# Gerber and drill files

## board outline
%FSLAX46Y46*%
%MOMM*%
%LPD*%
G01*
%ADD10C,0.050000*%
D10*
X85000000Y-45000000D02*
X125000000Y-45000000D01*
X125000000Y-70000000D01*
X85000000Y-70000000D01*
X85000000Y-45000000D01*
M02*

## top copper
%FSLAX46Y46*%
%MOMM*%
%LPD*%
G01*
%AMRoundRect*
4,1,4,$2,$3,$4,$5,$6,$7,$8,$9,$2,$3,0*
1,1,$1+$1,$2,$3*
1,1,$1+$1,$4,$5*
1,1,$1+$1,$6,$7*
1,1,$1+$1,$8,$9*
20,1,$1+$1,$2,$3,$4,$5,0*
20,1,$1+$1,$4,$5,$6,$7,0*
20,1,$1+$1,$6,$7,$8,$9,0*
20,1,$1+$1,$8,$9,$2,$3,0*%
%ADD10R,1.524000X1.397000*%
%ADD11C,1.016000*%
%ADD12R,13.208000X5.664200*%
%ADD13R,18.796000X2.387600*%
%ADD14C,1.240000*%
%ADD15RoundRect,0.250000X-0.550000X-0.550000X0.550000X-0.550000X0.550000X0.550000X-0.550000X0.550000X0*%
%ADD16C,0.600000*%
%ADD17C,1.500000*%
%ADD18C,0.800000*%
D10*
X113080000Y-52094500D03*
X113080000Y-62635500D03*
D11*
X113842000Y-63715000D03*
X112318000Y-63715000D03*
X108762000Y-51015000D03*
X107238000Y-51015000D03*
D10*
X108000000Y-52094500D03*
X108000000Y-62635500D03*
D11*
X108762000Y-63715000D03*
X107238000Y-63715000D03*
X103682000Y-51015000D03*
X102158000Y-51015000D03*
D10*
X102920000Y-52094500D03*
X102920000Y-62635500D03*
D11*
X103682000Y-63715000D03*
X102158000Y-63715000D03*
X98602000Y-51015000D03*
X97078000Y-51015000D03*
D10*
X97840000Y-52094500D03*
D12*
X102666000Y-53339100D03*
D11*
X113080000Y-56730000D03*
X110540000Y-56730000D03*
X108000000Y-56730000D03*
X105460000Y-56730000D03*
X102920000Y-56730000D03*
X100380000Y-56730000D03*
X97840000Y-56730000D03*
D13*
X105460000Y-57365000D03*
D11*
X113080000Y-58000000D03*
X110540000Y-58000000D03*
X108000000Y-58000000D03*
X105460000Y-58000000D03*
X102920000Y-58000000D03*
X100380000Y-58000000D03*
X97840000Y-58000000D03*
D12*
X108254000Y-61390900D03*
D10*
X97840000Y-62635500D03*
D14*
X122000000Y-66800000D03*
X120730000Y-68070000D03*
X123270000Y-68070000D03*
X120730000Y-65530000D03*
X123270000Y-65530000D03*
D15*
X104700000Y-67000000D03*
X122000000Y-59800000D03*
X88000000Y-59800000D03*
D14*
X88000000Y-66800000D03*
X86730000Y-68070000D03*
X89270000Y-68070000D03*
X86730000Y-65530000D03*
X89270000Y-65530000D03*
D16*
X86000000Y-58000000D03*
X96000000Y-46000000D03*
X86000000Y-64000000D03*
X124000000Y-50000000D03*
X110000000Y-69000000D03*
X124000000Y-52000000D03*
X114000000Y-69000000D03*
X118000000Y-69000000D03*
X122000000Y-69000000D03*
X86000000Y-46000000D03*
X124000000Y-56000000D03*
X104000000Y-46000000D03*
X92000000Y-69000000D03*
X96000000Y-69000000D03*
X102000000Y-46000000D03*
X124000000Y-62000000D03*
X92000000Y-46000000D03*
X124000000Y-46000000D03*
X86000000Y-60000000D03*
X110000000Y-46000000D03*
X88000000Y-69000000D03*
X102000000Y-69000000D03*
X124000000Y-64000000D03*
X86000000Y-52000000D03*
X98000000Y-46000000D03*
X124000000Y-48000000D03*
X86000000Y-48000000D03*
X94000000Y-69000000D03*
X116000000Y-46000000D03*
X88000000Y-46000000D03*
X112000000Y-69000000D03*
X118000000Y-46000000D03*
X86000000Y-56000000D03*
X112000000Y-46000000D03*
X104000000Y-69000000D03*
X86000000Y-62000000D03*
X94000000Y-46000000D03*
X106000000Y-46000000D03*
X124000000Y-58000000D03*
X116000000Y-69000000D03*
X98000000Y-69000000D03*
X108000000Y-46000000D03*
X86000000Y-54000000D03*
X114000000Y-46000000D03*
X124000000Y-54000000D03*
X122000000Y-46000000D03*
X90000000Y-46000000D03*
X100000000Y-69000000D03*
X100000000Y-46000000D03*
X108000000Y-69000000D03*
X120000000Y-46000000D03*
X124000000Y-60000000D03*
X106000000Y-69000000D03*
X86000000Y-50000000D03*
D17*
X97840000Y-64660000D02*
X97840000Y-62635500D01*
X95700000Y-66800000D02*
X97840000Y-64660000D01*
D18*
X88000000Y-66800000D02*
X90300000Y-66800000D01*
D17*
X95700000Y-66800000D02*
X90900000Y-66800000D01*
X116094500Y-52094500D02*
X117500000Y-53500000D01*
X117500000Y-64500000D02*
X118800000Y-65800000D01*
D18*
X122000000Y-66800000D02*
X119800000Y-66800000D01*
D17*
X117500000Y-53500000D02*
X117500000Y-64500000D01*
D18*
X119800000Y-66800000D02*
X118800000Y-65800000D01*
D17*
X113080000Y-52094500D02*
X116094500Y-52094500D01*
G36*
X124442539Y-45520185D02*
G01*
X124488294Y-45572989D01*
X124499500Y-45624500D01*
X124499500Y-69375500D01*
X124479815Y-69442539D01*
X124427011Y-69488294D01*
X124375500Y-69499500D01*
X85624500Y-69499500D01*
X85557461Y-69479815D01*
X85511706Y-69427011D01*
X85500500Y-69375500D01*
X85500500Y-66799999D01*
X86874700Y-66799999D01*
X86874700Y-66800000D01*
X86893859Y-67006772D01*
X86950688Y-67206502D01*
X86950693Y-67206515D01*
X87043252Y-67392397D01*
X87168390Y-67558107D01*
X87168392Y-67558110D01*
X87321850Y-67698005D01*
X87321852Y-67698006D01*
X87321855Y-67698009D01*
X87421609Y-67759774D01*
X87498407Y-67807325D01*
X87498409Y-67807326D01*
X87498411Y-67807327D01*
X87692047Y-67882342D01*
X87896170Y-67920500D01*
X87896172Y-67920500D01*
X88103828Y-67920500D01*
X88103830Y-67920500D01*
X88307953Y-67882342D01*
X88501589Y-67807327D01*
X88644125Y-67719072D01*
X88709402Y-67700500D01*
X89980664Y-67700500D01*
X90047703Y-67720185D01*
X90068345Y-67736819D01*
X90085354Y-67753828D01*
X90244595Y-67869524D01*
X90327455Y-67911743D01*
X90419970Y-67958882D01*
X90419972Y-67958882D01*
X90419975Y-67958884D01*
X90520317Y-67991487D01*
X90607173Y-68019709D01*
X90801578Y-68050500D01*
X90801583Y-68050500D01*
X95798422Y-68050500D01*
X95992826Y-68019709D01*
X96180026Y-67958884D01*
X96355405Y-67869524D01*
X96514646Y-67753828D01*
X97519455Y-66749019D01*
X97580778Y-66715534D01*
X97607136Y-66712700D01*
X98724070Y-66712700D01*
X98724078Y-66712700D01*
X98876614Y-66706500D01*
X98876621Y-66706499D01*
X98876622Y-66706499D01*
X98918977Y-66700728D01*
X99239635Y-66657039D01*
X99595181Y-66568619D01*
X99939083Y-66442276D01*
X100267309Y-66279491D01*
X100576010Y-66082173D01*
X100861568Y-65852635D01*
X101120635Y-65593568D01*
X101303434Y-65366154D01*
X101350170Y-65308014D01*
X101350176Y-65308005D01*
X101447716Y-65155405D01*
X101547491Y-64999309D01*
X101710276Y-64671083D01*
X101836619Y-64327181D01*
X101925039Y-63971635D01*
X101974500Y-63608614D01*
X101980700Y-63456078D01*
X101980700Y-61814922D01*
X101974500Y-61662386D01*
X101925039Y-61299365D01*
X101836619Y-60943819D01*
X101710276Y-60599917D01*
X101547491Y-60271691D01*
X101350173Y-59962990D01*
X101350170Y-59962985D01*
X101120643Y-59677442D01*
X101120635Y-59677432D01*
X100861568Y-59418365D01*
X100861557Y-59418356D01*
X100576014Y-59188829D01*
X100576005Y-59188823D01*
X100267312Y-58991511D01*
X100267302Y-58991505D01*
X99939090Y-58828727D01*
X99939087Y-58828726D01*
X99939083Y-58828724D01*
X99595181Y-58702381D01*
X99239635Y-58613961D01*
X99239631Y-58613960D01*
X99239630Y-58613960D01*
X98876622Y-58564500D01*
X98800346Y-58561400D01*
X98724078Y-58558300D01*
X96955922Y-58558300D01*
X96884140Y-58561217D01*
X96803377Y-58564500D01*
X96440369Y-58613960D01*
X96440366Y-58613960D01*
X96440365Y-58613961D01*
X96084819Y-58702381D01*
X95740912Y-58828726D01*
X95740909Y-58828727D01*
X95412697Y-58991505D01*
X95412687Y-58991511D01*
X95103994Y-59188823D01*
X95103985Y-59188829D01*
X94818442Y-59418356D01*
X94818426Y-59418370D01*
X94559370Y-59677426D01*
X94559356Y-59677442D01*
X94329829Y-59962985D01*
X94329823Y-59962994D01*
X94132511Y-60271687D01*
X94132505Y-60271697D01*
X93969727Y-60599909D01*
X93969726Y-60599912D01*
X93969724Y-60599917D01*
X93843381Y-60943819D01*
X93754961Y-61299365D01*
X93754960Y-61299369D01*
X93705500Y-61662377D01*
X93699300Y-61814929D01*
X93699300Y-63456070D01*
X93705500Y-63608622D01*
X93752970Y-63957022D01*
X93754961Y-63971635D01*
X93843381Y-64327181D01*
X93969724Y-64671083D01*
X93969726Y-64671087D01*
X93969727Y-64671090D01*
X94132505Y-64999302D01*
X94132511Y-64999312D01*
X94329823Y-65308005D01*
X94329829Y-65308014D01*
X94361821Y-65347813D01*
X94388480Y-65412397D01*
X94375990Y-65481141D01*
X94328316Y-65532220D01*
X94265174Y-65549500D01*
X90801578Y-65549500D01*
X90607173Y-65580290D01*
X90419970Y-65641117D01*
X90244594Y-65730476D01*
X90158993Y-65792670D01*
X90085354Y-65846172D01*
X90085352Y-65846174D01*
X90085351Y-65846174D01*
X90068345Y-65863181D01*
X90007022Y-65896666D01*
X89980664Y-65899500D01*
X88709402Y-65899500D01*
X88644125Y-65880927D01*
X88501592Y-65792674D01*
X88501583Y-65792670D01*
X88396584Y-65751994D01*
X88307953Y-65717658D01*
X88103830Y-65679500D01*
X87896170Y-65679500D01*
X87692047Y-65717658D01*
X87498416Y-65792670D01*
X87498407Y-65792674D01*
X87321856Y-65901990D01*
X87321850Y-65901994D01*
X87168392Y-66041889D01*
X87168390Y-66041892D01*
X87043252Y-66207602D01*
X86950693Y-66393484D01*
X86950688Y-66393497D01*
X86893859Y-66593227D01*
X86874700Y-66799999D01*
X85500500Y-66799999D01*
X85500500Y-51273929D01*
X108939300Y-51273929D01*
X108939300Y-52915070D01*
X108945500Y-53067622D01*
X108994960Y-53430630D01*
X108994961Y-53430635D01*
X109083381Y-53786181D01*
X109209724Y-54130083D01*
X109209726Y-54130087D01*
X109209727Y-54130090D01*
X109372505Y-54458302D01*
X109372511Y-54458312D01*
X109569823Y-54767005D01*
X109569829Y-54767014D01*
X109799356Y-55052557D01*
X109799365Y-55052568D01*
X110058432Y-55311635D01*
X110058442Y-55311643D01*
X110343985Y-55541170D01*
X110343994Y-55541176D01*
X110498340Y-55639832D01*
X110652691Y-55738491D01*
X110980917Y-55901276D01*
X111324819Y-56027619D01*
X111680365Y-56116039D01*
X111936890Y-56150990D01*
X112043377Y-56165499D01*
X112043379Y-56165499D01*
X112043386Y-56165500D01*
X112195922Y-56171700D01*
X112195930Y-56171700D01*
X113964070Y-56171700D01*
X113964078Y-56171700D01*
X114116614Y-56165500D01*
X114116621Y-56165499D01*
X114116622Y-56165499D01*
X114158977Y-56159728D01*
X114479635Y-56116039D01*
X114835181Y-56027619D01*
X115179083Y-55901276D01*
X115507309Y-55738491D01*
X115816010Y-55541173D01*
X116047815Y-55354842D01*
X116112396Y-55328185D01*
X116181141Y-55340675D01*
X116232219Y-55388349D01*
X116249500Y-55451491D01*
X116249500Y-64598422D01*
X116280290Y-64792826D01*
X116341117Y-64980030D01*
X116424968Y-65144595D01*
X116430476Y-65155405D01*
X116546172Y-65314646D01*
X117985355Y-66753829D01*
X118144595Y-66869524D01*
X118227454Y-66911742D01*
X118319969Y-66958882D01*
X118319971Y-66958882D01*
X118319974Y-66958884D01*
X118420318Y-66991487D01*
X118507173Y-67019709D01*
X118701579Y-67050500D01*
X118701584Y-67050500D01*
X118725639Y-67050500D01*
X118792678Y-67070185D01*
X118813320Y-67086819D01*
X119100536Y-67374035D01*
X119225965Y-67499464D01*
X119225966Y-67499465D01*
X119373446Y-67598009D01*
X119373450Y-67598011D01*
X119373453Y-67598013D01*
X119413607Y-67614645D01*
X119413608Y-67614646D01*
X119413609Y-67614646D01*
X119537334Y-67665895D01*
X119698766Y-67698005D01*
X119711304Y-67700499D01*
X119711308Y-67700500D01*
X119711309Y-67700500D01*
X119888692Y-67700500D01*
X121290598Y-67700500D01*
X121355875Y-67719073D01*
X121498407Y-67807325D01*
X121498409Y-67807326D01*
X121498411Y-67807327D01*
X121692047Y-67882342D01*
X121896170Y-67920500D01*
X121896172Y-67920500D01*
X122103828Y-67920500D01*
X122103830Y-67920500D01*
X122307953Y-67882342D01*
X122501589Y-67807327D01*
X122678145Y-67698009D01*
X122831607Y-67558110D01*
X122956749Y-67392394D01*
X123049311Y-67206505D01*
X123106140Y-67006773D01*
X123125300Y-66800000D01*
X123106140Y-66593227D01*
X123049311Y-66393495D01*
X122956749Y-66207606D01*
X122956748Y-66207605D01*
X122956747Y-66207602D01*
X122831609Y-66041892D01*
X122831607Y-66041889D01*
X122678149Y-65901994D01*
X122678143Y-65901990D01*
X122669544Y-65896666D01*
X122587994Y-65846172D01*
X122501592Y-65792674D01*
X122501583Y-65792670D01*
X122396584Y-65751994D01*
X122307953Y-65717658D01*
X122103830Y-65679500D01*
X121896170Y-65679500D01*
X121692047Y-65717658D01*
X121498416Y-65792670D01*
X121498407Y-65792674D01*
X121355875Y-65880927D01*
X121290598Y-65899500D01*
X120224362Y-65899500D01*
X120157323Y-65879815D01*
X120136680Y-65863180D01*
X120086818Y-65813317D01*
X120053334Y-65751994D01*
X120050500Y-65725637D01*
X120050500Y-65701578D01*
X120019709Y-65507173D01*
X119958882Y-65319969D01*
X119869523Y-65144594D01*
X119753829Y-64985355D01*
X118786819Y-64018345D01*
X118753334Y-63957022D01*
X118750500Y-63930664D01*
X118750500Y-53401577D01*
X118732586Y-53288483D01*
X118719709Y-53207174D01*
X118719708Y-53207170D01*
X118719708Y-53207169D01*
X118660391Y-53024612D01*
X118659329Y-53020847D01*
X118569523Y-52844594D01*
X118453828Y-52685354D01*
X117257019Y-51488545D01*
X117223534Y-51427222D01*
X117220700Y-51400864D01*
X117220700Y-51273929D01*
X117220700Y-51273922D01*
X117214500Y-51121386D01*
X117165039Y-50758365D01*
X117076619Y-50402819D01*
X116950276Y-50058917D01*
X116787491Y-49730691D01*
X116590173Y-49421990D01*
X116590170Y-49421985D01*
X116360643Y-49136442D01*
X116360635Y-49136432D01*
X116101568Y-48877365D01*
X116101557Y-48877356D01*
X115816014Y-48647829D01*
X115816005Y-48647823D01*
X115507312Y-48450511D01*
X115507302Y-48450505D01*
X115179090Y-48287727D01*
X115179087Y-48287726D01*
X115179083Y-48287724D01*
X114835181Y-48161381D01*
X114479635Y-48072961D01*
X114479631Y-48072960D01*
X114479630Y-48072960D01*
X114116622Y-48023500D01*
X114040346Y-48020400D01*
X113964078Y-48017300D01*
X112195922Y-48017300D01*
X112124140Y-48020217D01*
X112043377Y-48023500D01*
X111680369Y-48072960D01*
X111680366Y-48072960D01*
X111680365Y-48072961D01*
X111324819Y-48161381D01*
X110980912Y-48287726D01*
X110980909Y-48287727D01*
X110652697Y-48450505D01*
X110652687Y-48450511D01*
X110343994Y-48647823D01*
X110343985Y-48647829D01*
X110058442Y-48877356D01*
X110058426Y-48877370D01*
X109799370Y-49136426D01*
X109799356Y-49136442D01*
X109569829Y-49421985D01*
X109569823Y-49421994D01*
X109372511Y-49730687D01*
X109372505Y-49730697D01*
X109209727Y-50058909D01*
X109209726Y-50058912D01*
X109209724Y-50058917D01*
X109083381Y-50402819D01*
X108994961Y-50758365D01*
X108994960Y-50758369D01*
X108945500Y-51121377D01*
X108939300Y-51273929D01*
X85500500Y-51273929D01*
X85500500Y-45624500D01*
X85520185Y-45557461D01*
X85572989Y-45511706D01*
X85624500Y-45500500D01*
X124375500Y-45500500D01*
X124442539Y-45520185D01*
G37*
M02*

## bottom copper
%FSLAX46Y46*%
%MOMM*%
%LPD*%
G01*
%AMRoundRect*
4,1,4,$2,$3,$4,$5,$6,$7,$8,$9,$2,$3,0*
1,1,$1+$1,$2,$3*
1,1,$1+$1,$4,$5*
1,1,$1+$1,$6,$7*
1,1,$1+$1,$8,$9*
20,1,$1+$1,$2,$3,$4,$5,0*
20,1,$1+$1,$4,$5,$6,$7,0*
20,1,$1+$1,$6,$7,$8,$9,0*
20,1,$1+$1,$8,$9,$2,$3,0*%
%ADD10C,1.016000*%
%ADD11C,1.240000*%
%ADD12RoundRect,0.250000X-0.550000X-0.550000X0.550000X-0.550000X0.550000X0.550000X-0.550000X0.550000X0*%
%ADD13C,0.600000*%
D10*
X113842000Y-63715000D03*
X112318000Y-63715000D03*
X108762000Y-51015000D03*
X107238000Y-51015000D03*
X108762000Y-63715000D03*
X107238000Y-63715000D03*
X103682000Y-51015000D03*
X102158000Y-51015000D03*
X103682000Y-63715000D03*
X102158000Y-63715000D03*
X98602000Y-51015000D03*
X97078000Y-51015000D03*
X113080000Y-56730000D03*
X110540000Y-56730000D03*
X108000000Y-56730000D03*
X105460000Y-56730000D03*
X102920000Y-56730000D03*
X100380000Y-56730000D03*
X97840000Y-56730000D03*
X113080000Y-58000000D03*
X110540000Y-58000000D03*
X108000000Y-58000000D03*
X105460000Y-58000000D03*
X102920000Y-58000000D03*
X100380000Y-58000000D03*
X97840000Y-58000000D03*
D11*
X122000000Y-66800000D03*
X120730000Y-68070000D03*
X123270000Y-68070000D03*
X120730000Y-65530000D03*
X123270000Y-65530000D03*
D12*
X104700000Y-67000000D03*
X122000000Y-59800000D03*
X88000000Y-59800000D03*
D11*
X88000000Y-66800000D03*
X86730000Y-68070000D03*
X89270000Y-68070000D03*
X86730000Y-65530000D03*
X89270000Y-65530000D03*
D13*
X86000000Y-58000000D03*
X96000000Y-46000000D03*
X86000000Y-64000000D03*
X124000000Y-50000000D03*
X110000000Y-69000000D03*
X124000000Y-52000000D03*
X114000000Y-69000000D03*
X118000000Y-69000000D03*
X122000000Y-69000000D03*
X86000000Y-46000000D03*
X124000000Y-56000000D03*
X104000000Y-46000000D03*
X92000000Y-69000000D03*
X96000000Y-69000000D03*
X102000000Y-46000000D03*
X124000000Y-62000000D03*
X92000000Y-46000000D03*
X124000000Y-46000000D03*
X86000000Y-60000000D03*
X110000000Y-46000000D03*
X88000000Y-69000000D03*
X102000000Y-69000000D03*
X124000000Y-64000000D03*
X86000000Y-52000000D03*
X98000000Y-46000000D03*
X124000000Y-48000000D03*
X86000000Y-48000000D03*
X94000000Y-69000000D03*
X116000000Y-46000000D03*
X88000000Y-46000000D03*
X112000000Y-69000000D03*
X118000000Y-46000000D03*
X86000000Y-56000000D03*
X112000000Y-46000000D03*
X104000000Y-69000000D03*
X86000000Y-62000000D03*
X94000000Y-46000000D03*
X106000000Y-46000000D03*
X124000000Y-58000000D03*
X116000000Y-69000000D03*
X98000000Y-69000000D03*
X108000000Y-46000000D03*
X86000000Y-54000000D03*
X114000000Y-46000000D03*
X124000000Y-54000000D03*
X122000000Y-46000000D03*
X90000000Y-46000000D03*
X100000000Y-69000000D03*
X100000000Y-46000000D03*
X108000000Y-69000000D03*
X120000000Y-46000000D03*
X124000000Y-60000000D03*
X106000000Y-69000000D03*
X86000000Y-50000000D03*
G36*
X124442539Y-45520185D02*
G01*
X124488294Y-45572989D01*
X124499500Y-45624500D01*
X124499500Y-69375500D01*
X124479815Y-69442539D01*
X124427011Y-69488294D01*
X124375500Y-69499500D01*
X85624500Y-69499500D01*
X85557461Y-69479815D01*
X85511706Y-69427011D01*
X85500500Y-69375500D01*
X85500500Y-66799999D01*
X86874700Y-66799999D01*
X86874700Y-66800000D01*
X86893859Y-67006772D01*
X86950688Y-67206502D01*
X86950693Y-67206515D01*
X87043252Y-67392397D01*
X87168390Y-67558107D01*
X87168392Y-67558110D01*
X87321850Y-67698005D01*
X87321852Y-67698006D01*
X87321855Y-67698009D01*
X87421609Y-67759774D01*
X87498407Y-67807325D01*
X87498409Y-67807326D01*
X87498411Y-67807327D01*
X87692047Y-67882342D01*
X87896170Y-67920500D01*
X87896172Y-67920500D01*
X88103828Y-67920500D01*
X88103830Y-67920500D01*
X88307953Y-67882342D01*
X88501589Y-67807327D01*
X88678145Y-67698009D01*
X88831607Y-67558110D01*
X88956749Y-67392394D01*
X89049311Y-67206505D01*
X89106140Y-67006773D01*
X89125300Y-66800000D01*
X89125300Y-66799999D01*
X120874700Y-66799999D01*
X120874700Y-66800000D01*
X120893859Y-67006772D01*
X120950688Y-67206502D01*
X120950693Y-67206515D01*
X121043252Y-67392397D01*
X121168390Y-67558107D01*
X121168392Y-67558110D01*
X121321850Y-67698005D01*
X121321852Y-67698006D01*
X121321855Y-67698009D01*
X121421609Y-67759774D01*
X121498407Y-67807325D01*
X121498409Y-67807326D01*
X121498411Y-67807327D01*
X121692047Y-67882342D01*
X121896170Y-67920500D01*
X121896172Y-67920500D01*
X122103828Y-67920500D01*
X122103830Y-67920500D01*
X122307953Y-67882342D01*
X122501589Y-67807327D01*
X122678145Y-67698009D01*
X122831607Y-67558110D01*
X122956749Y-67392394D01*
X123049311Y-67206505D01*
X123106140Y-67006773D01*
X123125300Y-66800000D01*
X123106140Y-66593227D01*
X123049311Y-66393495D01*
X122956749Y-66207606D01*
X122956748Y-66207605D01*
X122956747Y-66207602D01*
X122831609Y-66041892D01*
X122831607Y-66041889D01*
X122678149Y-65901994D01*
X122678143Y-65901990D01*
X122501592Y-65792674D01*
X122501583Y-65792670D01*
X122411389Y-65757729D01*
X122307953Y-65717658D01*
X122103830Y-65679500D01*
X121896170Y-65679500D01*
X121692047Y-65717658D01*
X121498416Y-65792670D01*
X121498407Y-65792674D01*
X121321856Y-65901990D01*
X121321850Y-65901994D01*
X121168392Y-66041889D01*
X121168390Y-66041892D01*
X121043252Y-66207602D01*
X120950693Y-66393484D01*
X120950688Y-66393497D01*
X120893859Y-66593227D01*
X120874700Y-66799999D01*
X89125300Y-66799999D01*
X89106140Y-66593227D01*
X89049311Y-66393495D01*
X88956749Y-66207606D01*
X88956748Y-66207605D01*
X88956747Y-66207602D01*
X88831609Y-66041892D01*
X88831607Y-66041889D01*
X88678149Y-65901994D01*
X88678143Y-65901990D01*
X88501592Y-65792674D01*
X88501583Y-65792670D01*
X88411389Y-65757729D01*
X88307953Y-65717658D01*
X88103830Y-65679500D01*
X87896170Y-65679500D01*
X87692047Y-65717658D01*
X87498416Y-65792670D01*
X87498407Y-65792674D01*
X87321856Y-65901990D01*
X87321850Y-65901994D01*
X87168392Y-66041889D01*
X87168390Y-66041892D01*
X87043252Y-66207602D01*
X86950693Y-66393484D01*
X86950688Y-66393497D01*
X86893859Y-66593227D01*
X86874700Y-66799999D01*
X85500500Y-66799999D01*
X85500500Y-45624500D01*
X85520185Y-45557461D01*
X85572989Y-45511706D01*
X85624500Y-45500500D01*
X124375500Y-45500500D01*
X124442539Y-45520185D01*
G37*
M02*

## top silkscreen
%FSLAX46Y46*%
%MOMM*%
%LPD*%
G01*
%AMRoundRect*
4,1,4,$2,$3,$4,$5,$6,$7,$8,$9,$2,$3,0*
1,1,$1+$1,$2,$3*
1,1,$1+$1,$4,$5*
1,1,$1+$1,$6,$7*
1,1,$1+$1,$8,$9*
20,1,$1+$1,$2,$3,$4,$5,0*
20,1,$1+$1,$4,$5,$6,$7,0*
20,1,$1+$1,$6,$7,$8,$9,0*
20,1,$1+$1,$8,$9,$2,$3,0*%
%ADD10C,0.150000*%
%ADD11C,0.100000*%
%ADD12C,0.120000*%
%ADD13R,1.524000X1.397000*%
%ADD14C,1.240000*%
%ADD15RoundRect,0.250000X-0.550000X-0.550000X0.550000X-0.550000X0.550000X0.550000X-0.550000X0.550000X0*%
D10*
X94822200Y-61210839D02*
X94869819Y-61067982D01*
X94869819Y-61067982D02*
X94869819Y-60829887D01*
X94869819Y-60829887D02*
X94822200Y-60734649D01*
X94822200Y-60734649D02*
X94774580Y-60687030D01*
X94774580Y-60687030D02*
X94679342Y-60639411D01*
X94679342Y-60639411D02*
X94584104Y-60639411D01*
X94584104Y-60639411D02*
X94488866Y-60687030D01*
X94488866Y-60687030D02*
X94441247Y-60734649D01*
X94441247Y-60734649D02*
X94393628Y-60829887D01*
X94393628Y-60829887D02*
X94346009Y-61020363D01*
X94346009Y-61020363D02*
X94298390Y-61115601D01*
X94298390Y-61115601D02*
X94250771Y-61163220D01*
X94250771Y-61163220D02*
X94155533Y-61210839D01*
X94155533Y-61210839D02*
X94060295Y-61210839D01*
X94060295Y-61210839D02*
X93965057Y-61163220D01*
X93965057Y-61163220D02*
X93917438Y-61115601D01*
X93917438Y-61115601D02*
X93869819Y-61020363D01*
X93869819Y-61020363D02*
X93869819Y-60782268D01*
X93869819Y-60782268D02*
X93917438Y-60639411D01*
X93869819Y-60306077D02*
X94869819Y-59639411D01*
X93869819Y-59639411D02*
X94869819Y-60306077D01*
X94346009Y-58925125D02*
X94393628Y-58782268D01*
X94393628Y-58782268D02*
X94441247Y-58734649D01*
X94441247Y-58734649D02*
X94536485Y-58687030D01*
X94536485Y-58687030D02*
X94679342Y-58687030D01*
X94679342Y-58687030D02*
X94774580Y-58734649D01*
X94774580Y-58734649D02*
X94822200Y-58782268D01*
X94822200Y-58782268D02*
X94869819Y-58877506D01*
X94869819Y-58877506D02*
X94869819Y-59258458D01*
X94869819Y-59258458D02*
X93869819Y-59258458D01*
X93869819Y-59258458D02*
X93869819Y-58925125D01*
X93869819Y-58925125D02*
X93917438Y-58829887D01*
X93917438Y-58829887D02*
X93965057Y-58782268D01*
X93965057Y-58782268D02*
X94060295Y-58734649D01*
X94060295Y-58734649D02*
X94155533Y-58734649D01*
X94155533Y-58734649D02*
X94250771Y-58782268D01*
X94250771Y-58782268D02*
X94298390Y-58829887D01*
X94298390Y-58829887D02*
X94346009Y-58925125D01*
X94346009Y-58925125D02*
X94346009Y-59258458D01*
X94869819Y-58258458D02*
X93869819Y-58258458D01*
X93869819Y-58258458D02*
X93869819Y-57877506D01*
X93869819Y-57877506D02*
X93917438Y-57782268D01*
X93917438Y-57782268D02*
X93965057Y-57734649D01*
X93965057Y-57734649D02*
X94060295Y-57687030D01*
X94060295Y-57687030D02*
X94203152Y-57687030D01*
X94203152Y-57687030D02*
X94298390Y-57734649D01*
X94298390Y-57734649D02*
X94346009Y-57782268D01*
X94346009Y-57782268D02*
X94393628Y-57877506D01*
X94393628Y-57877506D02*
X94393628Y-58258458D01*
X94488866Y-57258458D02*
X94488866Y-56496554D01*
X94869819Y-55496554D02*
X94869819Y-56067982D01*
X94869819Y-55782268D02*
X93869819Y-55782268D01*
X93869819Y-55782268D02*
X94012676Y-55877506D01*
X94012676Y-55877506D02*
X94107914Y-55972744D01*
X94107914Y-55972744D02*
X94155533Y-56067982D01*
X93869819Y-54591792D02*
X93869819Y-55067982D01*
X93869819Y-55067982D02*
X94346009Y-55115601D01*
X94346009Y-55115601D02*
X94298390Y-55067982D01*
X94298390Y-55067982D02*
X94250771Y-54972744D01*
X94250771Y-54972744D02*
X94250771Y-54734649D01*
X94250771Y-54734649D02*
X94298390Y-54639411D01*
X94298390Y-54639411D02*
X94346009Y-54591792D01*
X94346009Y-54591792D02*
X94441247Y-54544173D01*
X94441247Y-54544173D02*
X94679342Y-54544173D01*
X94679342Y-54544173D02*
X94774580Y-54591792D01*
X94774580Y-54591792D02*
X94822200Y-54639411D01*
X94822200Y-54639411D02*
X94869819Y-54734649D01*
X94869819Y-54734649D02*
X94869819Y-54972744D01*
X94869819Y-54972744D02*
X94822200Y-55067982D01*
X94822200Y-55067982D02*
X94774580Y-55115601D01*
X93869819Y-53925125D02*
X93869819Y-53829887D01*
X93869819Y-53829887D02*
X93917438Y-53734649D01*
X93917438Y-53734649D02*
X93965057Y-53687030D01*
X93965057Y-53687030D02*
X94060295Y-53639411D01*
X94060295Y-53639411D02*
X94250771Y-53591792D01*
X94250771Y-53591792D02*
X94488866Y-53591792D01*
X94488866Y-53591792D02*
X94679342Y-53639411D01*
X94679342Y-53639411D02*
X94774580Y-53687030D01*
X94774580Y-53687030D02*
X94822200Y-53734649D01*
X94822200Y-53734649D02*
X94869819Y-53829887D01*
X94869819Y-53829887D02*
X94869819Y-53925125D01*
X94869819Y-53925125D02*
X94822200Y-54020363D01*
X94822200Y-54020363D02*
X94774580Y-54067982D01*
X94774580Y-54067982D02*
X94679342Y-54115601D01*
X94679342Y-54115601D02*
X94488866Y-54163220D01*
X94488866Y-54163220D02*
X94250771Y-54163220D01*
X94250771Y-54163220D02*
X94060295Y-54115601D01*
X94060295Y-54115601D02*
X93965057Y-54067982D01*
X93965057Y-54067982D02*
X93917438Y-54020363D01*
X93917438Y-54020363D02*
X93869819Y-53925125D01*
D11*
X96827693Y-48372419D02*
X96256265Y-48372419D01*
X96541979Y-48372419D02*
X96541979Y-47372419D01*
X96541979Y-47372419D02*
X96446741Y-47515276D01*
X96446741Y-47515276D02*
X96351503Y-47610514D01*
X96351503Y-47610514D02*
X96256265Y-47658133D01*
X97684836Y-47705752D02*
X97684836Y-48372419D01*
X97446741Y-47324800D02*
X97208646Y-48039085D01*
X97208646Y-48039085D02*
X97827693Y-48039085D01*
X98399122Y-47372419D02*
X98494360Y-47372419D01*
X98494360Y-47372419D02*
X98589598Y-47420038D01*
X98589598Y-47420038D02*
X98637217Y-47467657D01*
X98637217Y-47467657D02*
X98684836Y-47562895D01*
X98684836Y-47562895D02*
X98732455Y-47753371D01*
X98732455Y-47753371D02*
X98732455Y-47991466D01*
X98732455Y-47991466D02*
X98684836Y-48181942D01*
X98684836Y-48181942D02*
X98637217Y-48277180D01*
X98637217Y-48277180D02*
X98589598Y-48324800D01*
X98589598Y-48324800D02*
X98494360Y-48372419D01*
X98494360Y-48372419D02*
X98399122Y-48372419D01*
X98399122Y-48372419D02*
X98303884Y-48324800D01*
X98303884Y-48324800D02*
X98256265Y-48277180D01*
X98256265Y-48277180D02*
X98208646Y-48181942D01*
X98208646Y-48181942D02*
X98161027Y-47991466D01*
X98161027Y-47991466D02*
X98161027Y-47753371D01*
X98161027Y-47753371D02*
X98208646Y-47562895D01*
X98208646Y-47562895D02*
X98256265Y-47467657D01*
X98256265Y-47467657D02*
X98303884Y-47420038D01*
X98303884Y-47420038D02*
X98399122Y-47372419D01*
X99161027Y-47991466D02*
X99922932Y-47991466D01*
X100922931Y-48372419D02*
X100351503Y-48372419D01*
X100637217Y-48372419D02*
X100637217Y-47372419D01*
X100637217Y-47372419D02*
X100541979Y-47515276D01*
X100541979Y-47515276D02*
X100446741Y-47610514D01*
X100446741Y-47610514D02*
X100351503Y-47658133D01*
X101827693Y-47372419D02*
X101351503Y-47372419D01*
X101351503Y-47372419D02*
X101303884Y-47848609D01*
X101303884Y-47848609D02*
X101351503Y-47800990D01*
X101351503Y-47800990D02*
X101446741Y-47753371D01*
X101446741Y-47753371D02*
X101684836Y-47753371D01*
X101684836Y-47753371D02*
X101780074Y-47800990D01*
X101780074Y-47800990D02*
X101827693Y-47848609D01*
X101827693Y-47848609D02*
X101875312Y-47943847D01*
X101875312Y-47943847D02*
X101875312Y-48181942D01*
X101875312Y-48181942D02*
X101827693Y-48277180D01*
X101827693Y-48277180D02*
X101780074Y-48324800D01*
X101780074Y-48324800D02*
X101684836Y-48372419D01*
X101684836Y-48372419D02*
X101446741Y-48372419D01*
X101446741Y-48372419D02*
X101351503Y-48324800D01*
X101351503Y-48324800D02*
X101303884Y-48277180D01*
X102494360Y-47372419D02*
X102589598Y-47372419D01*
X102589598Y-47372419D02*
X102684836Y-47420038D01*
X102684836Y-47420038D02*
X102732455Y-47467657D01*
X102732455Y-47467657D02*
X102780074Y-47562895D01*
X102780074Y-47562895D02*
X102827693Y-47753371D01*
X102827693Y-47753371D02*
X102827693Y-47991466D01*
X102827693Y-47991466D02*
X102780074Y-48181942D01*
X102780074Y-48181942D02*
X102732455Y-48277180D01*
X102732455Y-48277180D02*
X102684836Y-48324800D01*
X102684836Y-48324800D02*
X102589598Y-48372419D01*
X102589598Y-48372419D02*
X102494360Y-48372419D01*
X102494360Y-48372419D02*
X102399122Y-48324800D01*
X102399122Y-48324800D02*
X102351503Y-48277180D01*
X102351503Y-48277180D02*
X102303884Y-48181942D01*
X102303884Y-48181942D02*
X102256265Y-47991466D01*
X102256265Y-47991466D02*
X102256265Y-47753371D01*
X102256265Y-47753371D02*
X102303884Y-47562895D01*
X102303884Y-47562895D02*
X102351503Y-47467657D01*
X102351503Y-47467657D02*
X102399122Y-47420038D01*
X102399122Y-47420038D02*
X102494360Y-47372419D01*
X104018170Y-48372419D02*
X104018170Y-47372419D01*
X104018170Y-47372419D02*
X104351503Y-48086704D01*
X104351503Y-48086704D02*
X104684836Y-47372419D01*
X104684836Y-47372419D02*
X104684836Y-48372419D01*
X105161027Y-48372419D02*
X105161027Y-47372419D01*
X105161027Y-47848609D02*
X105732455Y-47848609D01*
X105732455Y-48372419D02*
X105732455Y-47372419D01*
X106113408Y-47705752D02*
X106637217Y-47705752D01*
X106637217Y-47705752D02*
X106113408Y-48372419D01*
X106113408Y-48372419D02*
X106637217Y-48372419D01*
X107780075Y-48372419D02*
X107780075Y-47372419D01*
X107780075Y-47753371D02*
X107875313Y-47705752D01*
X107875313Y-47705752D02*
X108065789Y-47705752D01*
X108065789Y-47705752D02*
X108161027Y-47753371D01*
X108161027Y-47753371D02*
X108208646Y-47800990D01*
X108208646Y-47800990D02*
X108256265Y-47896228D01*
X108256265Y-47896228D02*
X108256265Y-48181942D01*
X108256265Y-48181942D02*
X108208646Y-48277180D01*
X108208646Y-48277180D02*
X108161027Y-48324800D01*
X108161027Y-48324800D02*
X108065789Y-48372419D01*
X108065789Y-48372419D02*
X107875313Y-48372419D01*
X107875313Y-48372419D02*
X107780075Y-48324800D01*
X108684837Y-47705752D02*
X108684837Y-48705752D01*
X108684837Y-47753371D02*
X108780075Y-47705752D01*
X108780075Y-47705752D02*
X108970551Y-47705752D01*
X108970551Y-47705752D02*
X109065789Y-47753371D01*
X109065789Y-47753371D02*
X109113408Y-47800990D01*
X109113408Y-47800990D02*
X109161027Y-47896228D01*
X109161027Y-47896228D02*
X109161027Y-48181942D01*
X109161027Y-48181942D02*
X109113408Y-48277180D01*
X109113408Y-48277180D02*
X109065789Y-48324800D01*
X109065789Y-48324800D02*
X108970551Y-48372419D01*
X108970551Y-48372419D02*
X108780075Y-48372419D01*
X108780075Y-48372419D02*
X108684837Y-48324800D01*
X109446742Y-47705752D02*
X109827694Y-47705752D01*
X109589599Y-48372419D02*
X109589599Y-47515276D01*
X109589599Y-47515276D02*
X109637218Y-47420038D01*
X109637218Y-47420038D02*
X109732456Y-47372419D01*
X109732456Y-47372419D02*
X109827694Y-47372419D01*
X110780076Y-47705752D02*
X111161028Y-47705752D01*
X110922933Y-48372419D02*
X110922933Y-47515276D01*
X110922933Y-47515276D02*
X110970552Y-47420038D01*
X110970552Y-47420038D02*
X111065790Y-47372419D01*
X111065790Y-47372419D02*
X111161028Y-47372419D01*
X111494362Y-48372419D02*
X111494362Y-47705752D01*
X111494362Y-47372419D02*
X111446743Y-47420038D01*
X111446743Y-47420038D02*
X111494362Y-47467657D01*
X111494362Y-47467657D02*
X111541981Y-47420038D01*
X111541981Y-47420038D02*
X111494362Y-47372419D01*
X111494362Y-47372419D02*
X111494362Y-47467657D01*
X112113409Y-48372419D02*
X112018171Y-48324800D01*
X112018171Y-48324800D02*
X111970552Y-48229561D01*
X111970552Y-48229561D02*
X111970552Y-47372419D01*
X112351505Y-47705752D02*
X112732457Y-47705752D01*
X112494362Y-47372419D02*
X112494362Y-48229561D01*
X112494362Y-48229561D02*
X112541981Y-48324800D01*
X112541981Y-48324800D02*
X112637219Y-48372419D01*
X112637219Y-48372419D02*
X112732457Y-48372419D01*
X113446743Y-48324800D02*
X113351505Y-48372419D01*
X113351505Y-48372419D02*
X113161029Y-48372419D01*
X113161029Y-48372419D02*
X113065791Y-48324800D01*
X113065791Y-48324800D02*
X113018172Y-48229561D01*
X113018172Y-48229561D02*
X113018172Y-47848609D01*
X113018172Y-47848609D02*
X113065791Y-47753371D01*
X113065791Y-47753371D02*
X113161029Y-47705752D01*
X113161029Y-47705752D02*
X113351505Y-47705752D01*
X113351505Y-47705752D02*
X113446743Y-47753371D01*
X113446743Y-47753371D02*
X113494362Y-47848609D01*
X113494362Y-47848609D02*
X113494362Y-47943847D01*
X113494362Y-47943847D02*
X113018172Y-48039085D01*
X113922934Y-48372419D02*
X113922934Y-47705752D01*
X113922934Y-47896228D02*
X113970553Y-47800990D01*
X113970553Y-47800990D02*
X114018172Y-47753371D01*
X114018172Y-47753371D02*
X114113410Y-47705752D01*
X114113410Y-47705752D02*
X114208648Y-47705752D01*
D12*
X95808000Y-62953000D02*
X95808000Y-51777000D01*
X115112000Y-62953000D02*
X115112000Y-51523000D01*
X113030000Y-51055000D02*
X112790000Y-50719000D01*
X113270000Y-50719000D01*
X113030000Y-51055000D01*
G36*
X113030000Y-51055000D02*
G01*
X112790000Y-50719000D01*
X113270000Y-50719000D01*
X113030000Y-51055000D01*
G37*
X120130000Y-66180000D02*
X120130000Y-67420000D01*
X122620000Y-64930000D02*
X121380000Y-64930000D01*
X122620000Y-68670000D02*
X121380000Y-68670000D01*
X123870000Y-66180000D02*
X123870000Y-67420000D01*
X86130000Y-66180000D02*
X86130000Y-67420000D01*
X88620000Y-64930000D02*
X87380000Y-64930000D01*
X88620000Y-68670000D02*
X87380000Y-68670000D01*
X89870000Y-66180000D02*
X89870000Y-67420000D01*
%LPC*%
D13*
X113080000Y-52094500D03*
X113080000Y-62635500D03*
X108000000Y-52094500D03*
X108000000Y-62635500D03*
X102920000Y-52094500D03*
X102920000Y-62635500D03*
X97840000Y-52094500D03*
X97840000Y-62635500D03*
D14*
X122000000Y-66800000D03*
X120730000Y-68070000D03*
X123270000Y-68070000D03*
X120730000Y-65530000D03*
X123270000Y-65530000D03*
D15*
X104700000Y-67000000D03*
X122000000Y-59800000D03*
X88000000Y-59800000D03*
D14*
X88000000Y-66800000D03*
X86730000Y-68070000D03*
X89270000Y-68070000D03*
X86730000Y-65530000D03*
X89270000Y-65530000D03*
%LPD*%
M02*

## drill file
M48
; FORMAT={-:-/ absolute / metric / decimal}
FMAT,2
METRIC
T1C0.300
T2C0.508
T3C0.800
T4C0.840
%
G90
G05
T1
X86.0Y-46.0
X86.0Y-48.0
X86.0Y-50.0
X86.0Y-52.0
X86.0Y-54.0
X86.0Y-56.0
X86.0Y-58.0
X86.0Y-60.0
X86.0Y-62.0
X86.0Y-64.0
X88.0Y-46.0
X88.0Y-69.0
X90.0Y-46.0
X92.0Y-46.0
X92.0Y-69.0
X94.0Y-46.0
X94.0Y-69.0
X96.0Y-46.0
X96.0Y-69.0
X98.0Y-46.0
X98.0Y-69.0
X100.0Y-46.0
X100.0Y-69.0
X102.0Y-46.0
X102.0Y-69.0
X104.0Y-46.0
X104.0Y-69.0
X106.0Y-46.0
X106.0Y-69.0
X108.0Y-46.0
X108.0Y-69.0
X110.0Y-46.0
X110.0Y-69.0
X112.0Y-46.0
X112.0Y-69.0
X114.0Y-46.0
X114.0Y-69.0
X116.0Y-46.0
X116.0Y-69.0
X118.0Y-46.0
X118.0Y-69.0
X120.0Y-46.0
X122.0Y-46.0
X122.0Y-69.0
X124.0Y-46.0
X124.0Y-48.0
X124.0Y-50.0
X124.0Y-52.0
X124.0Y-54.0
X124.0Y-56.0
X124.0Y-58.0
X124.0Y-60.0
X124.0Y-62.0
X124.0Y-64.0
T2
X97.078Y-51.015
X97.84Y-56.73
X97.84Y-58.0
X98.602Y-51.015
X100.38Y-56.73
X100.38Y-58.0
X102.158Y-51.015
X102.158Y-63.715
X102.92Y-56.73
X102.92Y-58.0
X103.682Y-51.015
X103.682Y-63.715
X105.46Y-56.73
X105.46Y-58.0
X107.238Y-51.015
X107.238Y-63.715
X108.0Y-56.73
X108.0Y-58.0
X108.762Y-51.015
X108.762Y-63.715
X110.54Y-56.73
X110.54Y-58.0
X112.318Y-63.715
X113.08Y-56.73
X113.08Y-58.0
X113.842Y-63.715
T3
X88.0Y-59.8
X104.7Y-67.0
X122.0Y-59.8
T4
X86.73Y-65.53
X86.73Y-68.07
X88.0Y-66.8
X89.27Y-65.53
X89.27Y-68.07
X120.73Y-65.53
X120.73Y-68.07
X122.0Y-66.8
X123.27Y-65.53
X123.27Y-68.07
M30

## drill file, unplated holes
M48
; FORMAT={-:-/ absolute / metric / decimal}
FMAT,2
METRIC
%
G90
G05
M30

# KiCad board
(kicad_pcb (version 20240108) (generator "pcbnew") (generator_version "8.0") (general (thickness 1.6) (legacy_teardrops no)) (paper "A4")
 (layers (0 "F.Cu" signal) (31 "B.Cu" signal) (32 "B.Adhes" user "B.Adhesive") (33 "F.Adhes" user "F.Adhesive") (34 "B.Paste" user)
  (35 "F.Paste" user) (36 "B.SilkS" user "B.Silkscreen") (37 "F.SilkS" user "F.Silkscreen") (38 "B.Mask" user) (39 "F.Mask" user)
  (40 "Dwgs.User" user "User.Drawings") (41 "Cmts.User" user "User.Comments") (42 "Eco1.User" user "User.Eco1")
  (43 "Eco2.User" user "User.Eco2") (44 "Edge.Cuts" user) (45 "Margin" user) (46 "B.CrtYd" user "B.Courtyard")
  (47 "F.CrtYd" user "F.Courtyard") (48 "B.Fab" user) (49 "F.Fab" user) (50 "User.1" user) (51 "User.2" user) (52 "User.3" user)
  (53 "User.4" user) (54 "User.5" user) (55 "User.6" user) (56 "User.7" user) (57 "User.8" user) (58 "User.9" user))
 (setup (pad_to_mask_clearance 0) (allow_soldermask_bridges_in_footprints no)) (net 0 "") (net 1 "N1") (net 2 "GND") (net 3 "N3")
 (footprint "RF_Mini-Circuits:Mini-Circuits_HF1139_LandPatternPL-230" (layer "F.Cu") (at 105.46 57.365 -90)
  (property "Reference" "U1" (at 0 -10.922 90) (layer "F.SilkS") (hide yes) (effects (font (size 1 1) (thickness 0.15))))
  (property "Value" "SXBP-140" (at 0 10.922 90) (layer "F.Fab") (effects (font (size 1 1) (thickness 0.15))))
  (fp_line (start 5.588 9.652) (end -5.588 9.652) (stroke (width 0.12) (type solid)) (layer "F.SilkS"))
  (fp_line (start 5.588 -9.652) (end -5.842 -9.652) (stroke (width 0.12) (type solid)) (layer "F.SilkS"))
  (fp_poly
   (pts (xy -6.31 -7.57) (xy -6.646 -7.33) (xy -6.646 -7.81) (xy -6.31 -7.57)) (stroke (width 0.12) (type solid)) (fill solid)
   (layer "F.SilkS"))
  (pad "1" smd rect (at -5.2705 -7.62 180) (size 1.524 1.397) (layers "F.Cu" "F.Paste" "F.Mask") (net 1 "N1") (clearance 3.3782))
  (pad "2" smd rect (at 5.2705 -7.62 180) (size 1.524 1.397) (layers "F.Cu" "F.Paste" "F.Mask") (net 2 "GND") (zone_connect 2))
  (pad "2" thru_hole circle (at 6.35 -8.382 180) (size 1.016 1.016) (drill 0.508) (layers "*.Cu") (remove_unused_layers no) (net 2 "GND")
   (zone_connect 2))
  (pad "2" thru_hole circle (at 6.35 -6.858 180) (size 1.016 1.016) (drill 0.508) (layers "*.Cu") (remove_unused_layers no) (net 2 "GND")
   (zone_connect 2))
  (pad "3" thru_hole circle (at -6.35 -3.302 180) (size 1.016 1.016) (drill 0.508) (layers "*.Cu") (remove_unused_layers no) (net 2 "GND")
   (zone_connect 2))
  (pad "3" thru_hole circle (at -6.35 -1.778 180) (size 1.016 1.016) (drill 0.508) (layers "*.Cu") (remove_unused_layers no) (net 2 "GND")
   (zone_connect 2))
  (pad "3" smd rect (at -5.2705 -2.54 180) (size 1.524 1.397) (layers "F.Cu" "F.Paste" "F.Mask") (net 2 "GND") (zone_connect 2))
  (pad "4" smd rect (at 5.2705 -2.54 180) (size 1.524 1.397) (layers "F.Cu" "F.Paste" "F.Mask") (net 2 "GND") (zone_connect 2))
  (pad "4" thru_hole circle (at 6.35 -3.302 180) (size 1.016 1.016) (drill 0.508) (layers "*.Cu") (remove_unused_layers no) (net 2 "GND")
   (zone_connect 2))
  (pad "4" thru_hole circle (at 6.35 -1.778 180) (size 1.016 1.016) (drill 0.508) (layers "*.Cu") (remove_unused_layers no) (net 2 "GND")
   (zone_connect 2))
  (pad "5" thru_hole circle (at -6.35 1.778 180) (size 1.016 1.016) (drill 0.508) (layers "*.Cu") (remove_unused_layers no) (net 2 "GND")
   (zone_connect 2))
  (pad "5" thru_hole circle (at -6.35 3.302 180) (size 1.016 1.016) (drill 0.508) (layers "*.Cu") (remove_unused_layers no) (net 2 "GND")
   (zone_connect 2))
  (pad "5" smd rect (at -5.2705 2.54 180) (size 1.524 1.397) (layers "F.Cu" "F.Paste" "F.Mask") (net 2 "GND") (zone_connect 2))
  (pad "6" smd rect (at 5.2705 2.54 180) (size 1.524 1.397) (layers "F.Cu" "F.Paste" "F.Mask") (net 2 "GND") (zone_connect 2))
  (pad "6" thru_hole circle (at 6.35 1.778 180) (size 1.016 1.016) (drill 0.508) (layers "*.Cu") (remove_unused_layers no) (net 2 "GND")
   (zone_connect 2))
  (pad "6" thru_hole circle (at 6.35 3.302 180) (size 1.016 1.016) (drill 0.508) (layers "*.Cu") (remove_unused_layers no) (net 2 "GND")
   (zone_connect 2))
  (pad "7" thru_hole circle (at -6.35 6.858 180) (size 1.016 1.016) (drill 0.508) (layers "*.Cu") (remove_unused_layers no) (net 2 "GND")
   (zone_connect 2))
  (pad "7" thru_hole circle (at -6.35 8.382 180) (size 1.016 1.016) (drill 0.508) (layers "*.Cu") (remove_unused_layers no) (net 2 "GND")
   (zone_connect 2))
  (pad "7" smd rect (at -5.2705 7.62 180) (size 1.524 1.397) (layers "F.Cu" "F.Paste" "F.Mask") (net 2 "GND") (zone_connect 2))
  (pad "7" smd rect (at -4.0259 2.794 180) (size 13.208 5.6642) (layers "F.Cu") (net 2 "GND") (zone_connect 2))
  (pad "7" thru_hole circle (at -0.635 -7.62 180) (size 1.016 1.016) (drill 0.508) (layers "*.Cu") (remove_unused_layers no) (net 2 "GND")
   (zone_connect 2))
  (pad "7" thru_hole circle (at -0.635 -5.08 180) (size 1.016 1.016) (drill 0.508) (layers "*.Cu") (remove_unused_layers no) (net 2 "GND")
   (zone_connect 2))
  (pad "7" thru_hole circle (at -0.635 -2.54 180) (size 1.016 1.016) (drill 0.508) (layers "*.Cu") (remove_unused_layers no) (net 2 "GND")
   (zone_connect 2))
  (pad "7" thru_hole circle (at -0.635 0 180) (size 1.016 1.016) (drill 0.508) (layers "*.Cu") (remove_unused_layers no) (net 2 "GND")
   (zone_connect 2))
  (pad "7" thru_hole circle (at -0.635 2.54 180) (size 1.016 1.016) (drill 0.508) (layers "*.Cu") (remove_unused_layers no) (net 2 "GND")
   (zone_connect 2))
  (pad "7" thru_hole circle (at -0.635 5.08 180) (size 1.016 1.016) (drill 0.508) (layers "*.Cu") (remove_unused_layers no) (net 2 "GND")
   (zone_connect 2))
  (pad "7" thru_hole circle (at -0.635 7.62 180) (size 1.016 1.016) (drill 0.508) (layers "*.Cu") (remove_unused_layers no) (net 2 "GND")
   (zone_connect 2))
  (pad "7" smd rect (at 0 0 180) (size 18.796 2.3876) (layers "F.Cu") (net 2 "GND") (zone_connect 2))
  (pad "7" thru_hole circle (at 0.635 -7.62 180) (size 1.016 1.016) (drill 0.508) (layers "*.Cu") (remove_unused_layers no) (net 2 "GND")
   (zone_connect 2))
  (pad "7" thru_hole circle (at 0.635 -5.08 180) (size 1.016 1.016) (drill 0.508) (layers "*.Cu") (remove_unused_layers no) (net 2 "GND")
   (zone_connect 2))
  (pad "7" thru_hole circle (at 0.635 -2.54 180) (size 1.016 1.016) (drill 0.508) (layers "*.Cu") (remove_unused_layers no) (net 2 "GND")
   (zone_connect 2))
  (pad "7" thru_hole circle (at 0.635 0 180) (size 1.016 1.016) (drill 0.508) (layers "*.Cu") (remove_unused_layers no) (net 2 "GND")
   (zone_connect 2))
  (pad "7" thru_hole circle (at 0.635 2.54 180) (size 1.016 1.016) (drill 0.508) (layers "*.Cu") (remove_unused_layers no) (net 2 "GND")
   (zone_connect 2))
  (pad "7" thru_hole circle (at 0.635 5.08 180) (size 1.016 1.016) (drill 0.508) (layers "*.Cu") (remove_unused_layers no) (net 2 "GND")
   (zone_connect 2))
  (pad "7" thru_hole circle (at 0.635 7.62 180) (size 1.016 1.016) (drill 0.508) (layers "*.Cu") (remove_unused_layers no) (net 2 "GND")
   (zone_connect 2))
  (pad "7" smd rect (at 4.0259 -2.794 180) (size 13.208 5.6642) (layers "F.Cu") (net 2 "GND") (zone_connect 2))
  (pad "8" smd rect (at 5.2705 7.62 180) (size 1.524 1.397) (layers "F.Cu" "F.Paste" "F.Mask") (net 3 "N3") (clearance 3.3782)))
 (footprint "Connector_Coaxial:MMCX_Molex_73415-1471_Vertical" (layer "F.Cu") (at 122 66.8 90)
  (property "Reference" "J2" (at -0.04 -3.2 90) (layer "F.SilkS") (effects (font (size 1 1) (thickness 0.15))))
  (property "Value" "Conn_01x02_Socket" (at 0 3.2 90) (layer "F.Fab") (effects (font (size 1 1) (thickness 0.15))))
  (fp_line (start 0.62 -1.87) (end -0.62 -1.87) (stroke (width 0.12) (type solid)) (layer "F.SilkS"))
  (fp_line (start 1.87 0.62) (end 1.87 -0.62) (stroke (width 0.12) (type solid)) (layer "F.SilkS"))
  (fp_line (start -1.87 0.62) (end -1.87 -0.62) (stroke (width 0.12) (type solid)) (layer "F.SilkS"))
  (fp_line (start 0.62 1.87) (end -0.62 1.87) (stroke (width 0.12) (type solid)) (layer "F.SilkS"))
  (pad "1" thru_hole circle (at 0 0 90) (size 1.24 1.24) (drill 0.84) (layers "*.Cu" "*.Mask") (remove_unused_layers no) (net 1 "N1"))
  (pad "2" thru_hole circle (at -1.27 -1.27 90) (size 1.24 1.24) (drill 0.84) (layers "*.Cu" "*.Mask") (remove_unused_layers no)
   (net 2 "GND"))
  (pad "2" thru_hole circle (at -1.27 1.27 90) (size 1.24 1.24) (drill 0.84) (layers "*.Cu" "*.Mask") (remove_unused_layers no)
   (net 2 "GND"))
  (pad "2" thru_hole circle (at 1.27 -1.27 90) (size 1.24 1.24) (drill 0.84) (layers "*.Cu" "*.Mask") (remove_unused_layers no)
   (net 2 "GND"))
  (pad "2" thru_hole circle (at 1.27 1.27 90) (size 1.24 1.24) (drill 0.84) (layers "*.Cu" "*.Mask") (remove_unused_layers no) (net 2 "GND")))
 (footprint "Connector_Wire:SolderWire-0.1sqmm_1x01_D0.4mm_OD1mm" (layer "F.Cu") (at 104.7 67)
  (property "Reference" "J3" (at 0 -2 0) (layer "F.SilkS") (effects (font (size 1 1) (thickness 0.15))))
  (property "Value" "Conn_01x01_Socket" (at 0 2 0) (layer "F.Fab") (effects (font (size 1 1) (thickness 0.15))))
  (pad "1" thru_hole roundrect (at 0 0) (size 1.6 1.6) (drill 0.8) (layers "*.Cu" "*.Mask") (remove_unused_layers no)
   (roundrect_rratio 0.15625) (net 2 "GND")))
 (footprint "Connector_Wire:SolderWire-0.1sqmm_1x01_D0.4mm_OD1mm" (layer "F.Cu") (at 71.1 59.7)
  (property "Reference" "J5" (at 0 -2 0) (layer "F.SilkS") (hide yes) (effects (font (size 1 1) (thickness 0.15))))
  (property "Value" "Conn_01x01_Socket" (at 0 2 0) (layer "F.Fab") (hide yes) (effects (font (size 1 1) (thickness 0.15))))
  (pad "1" thru_hole roundrect (at 50.9 0.1) (size 1.6 1.6) (drill 0.8) (layers "*.Cu" "*.Mask") (remove_unused_layers no)
   (roundrect_rratio 0.15625) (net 2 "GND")))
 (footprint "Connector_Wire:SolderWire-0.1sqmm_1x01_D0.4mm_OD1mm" (layer "F.Cu") (at 71.1 56.05)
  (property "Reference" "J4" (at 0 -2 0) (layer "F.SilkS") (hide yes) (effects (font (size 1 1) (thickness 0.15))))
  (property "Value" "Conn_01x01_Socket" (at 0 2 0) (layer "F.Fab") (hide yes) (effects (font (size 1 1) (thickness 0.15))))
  (pad "1" thru_hole roundrect (at 16.9 3.75) (size 1.6 1.6) (drill 0.8) (layers "*.Cu" "*.Mask") (remove_unused_layers no)
   (roundrect_rratio 0.15625) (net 2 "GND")))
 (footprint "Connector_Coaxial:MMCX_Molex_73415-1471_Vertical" (layer "F.Cu") (at 88 66.8 90)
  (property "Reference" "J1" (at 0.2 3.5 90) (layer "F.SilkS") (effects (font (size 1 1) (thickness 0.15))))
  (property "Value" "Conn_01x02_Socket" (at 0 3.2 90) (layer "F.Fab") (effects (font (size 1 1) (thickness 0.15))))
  (fp_line (start 0.62 -1.87) (end -0.62 -1.87) (stroke (width 0.12) (type solid)) (layer "F.SilkS"))
  (fp_line (start 1.87 0.62) (end 1.87 -0.62) (stroke (width 0.12) (type solid)) (layer "F.SilkS"))
  (fp_line (start -1.87 0.62) (end -1.87 -0.62) (stroke (width 0.12) (type solid)) (layer "F.SilkS"))
  (fp_line (start 0.62 1.87) (end -0.62 1.87) (stroke (width 0.12) (type solid)) (layer "F.SilkS"))
  (pad "1" thru_hole circle (at 0 0 90) (size 1.24 1.24) (drill 0.84) (layers "*.Cu" "*.Mask") (remove_unused_layers no) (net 3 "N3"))
  (pad "2" thru_hole circle (at -1.27 -1.27 90) (size 1.24 1.24) (drill 0.84) (layers "*.Cu" "*.Mask") (remove_unused_layers no)
   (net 2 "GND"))
  (pad "2" thru_hole circle (at -1.27 1.27 90) (size 1.24 1.24) (drill 0.84) (layers "*.Cu" "*.Mask") (remove_unused_layers no)
   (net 2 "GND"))
  (pad "2" thru_hole circle (at 1.27 -1.27 90) (size 1.24 1.24) (drill 0.84) (layers "*.Cu" "*.Mask") (remove_unused_layers no)
   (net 2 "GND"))
  (pad "2" thru_hole circle (at 1.27 1.27 90) (size 1.24 1.24) (drill 0.84) (layers "*.Cu" "*.Mask") (remove_unused_layers no) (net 2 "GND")))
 (gr_rect (start 85 45) (end 125 70) (stroke (width 0.05) (type default)) (fill none) (layer "Edge.Cuts"))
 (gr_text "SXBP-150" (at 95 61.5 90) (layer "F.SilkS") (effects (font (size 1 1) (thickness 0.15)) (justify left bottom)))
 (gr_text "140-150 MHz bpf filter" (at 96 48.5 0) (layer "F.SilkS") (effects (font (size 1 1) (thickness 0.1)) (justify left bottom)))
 (segment (start 97.84 64.66) (end 97.84 62.6355) (width 1.5) (layer "F.Cu") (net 3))
 (segment (start 95.7 66.8) (end 97.84 64.66) (width 1.5) (layer "F.Cu") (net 3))
 (segment (start 88 66.8) (end 90.3 66.8) (width 0.8) (layer "F.Cu") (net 3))
 (segment (start 95.7 66.8) (end 90.9 66.8) (width 1.5) (layer "F.Cu") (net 3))
 (via (at 86 58) (size 0.6) (drill 0.3) (layers "F.Cu" "B.Cu") (free yes) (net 2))
 (via (at 96 46) (size 0.6) (drill 0.3) (layers "F.Cu" "B.Cu") (free yes) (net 2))
 (via (at 86 64) (size 0.6) (drill 0.3) (layers "F.Cu" "B.Cu") (free yes) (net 2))
 (via (at 124 50) (size 0.6) (drill 0.3) (layers "F.Cu" "B.Cu") (free yes) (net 2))
 (via (at 110 69) (size 0.6) (drill 0.3) (layers "F.Cu" "B.Cu") (free yes) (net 2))
 (via (at 124 52) (size 0.6) (drill 0.3) (layers "F.Cu" "B.Cu") (free yes) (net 2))
 (via (at 114 69) (size 0.6) (drill 0.3) (layers "F.Cu" "B.Cu") (free yes) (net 2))
 (via (at 118 69) (size 0.6) (drill 0.3) (layers "F.Cu" "B.Cu") (free yes) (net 2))
 (via (at 122 69) (size 0.6) (drill 0.3) (layers "F.Cu" "B.Cu") (free yes) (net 2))
 (via (at 86 46) (size 0.6) (drill 0.3) (layers "F.Cu" "B.Cu") (free yes) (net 2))
 (via (at 124 56) (size 0.6) (drill 0.3) (layers "F.Cu" "B.Cu") (free yes) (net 2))
 (via (at 104 46) (size 0.6) (drill 0.3) (layers "F.Cu" "B.Cu") (free yes) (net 2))
 (via (at 92 69) (size 0.6) (drill 0.3) (layers "F.Cu" "B.Cu") (free yes) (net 2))
 (via (at 96 69) (size 0.6) (drill 0.3) (layers "F.Cu" "B.Cu") (free yes) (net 2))
 (via (at 102 46) (size 0.6) (drill 0.3) (layers "F.Cu" "B.Cu") (free yes) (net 2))
 (via (at 124 62) (size 0.6) (drill 0.3) (layers "F.Cu" "B.Cu") (free yes) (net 2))
 (via (at 92 46) (size 0.6) (drill 0.3) (layers "F.Cu" "B.Cu") (free yes) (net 2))
 (via (at 124 46) (size 0.6) (drill 0.3) (layers "F.Cu" "B.Cu") (free yes) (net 2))
 (via (at 86 60) (size 0.6) (drill 0.3) (layers "F.Cu" "B.Cu") (free yes) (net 2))
 (via (at 110 46) (size 0.6) (drill 0.3) (layers "F.Cu" "B.Cu") (free yes) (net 2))
 (via (at 88 69) (size 0.6) (drill 0.3) (layers "F.Cu" "B.Cu") (free yes) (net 2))
 (via (at 102 69) (size 0.6) (drill 0.3) (layers "F.Cu" "B.Cu") (free yes) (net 2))
 (via (at 124 64) (size 0.6) (drill 0.3) (layers "F.Cu" "B.Cu") (free yes) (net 2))
 (via (at 86 52) (size 0.6) (drill 0.3) (layers "F.Cu" "B.Cu") (free yes) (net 2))
 (via (at 98 46) (size 0.6) (drill 0.3) (layers "F.Cu" "B.Cu") (free yes) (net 2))
 (via (at 124 48) (size 0.6) (drill 0.3) (layers "F.Cu" "B.Cu") (free yes) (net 2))
 (via (at 86 48) (size 0.6) (drill 0.3) (layers "F.Cu" "B.Cu") (free yes) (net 2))
 (via (at 94 69) (size 0.6) (drill 0.3) (layers "F.Cu" "B.Cu") (free yes) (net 2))
 (via (at 116 46) (size 0.6) (drill 0.3) (layers "F.Cu" "B.Cu") (free yes) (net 2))
 (via (at 88 46) (size 0.6) (drill 0.3) (layers "F.Cu" "B.Cu") (free yes) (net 2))
 (via (at 112 69) (size 0.6) (drill 0.3) (layers "F.Cu" "B.Cu") (free yes) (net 2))
 (via (at 118 46) (size 0.6) (drill 0.3) (layers "F.Cu" "B.Cu") (free yes) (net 2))
 (via (at 86 56) (size 0.6) (drill 0.3) (layers "F.Cu" "B.Cu") (free yes) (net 2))
 (via (at 112 46) (size 0.6) (drill 0.3) (layers "F.Cu" "B.Cu") (free yes) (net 2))
 (via (at 104 69) (size 0.6) (drill 0.3) (layers "F.Cu" "B.Cu") (free yes) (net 2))
 (via (at 86 62) (size 0.6) (drill 0.3) (layers "F.Cu" "B.Cu") (free yes) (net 2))
 (via (at 94 46) (size 0.6) (drill 0.3) (layers "F.Cu" "B.Cu") (free yes) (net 2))
 (via (at 106 46) (size 0.6) (drill 0.3) (layers "F.Cu" "B.Cu") (free yes) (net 2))
 (via (at 124 58) (size 0.6) (drill 0.3) (layers "F.Cu" "B.Cu") (free yes) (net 2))
 (via (at 116 69) (size 0.6) (drill 0.3) (layers "F.Cu" "B.Cu") (free yes) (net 2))
 (via (at 98 69) (size 0.6) (drill 0.3) (layers "F.Cu" "B.Cu") (free yes) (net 2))
 (via (at 108 46) (size 0.6) (drill 0.3) (layers "F.Cu" "B.Cu") (free yes) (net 2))
 (via (at 86 54) (size 0.6) (drill 0.3) (layers "F.Cu" "B.Cu") (free yes) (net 2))
 (via (at 114 46) (size 0.6) (drill 0.3) (layers "F.Cu" "B.Cu") (free yes) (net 2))
 (via (at 124 54) (size 0.6) (drill 0.3) (layers "F.Cu" "B.Cu") (free yes) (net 2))
 (via (at 122 46) (size 0.6) (drill 0.3) (layers "F.Cu" "B.Cu") (free yes) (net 2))
 (via (at 90 46) (size 0.6) (drill 0.3) (layers "F.Cu" "B.Cu") (free yes) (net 2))
 (via (at 100 69) (size 0.6) (drill 0.3) (layers "F.Cu" "B.Cu") (free yes) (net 2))
 (via (at 100 46) (size 0.6) (drill 0.3) (layers "F.Cu" "B.Cu") (free yes) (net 2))
 (via (at 108 69) (size 0.6) (drill 0.3) (layers "F.Cu" "B.Cu") (free yes) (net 2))
 (via (at 120 46) (size 0.6) (drill 0.3) (layers "F.Cu" "B.Cu") (free yes) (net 2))
 (via (at 124 60) (size 0.6) (drill 0.3) (layers "F.Cu" "B.Cu") (free yes) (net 2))
 (via (at 106 69) (size 0.6) (drill 0.3) (layers "F.Cu" "B.Cu") (free yes) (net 2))
 (via (at 86 50) (size 0.6) (drill 0.3) (layers "F.Cu" "B.Cu") (free yes) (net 2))
 (segment (start 116.0945 52.0945) (end 117.5 53.5) (width 1.5) (layer "F.Cu") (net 1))
 (segment (start 117.5 64.5) (end 118.8 65.8) (width 1.5) (layer "F.Cu") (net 1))
 (segment (start 122 66.8) (end 119.8 66.8) (width 0.8) (layer "F.Cu") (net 1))
 (segment (start 117.5 53.5) (end 117.5 64.5) (width 1.5) (layer "F.Cu") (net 1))
 (segment (start 119.8 66.8) (end 118.8 65.8) (width 0.8) (layer "F.Cu") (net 1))
 (segment (start 113.08 52.0945) (end 116.0945 52.0945) (width 1.5) (layer "F.Cu") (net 1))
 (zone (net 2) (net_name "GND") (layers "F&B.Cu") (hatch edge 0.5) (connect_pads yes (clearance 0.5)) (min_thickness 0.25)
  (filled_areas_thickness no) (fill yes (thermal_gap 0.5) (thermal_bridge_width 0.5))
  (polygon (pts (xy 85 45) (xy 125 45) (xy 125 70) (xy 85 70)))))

